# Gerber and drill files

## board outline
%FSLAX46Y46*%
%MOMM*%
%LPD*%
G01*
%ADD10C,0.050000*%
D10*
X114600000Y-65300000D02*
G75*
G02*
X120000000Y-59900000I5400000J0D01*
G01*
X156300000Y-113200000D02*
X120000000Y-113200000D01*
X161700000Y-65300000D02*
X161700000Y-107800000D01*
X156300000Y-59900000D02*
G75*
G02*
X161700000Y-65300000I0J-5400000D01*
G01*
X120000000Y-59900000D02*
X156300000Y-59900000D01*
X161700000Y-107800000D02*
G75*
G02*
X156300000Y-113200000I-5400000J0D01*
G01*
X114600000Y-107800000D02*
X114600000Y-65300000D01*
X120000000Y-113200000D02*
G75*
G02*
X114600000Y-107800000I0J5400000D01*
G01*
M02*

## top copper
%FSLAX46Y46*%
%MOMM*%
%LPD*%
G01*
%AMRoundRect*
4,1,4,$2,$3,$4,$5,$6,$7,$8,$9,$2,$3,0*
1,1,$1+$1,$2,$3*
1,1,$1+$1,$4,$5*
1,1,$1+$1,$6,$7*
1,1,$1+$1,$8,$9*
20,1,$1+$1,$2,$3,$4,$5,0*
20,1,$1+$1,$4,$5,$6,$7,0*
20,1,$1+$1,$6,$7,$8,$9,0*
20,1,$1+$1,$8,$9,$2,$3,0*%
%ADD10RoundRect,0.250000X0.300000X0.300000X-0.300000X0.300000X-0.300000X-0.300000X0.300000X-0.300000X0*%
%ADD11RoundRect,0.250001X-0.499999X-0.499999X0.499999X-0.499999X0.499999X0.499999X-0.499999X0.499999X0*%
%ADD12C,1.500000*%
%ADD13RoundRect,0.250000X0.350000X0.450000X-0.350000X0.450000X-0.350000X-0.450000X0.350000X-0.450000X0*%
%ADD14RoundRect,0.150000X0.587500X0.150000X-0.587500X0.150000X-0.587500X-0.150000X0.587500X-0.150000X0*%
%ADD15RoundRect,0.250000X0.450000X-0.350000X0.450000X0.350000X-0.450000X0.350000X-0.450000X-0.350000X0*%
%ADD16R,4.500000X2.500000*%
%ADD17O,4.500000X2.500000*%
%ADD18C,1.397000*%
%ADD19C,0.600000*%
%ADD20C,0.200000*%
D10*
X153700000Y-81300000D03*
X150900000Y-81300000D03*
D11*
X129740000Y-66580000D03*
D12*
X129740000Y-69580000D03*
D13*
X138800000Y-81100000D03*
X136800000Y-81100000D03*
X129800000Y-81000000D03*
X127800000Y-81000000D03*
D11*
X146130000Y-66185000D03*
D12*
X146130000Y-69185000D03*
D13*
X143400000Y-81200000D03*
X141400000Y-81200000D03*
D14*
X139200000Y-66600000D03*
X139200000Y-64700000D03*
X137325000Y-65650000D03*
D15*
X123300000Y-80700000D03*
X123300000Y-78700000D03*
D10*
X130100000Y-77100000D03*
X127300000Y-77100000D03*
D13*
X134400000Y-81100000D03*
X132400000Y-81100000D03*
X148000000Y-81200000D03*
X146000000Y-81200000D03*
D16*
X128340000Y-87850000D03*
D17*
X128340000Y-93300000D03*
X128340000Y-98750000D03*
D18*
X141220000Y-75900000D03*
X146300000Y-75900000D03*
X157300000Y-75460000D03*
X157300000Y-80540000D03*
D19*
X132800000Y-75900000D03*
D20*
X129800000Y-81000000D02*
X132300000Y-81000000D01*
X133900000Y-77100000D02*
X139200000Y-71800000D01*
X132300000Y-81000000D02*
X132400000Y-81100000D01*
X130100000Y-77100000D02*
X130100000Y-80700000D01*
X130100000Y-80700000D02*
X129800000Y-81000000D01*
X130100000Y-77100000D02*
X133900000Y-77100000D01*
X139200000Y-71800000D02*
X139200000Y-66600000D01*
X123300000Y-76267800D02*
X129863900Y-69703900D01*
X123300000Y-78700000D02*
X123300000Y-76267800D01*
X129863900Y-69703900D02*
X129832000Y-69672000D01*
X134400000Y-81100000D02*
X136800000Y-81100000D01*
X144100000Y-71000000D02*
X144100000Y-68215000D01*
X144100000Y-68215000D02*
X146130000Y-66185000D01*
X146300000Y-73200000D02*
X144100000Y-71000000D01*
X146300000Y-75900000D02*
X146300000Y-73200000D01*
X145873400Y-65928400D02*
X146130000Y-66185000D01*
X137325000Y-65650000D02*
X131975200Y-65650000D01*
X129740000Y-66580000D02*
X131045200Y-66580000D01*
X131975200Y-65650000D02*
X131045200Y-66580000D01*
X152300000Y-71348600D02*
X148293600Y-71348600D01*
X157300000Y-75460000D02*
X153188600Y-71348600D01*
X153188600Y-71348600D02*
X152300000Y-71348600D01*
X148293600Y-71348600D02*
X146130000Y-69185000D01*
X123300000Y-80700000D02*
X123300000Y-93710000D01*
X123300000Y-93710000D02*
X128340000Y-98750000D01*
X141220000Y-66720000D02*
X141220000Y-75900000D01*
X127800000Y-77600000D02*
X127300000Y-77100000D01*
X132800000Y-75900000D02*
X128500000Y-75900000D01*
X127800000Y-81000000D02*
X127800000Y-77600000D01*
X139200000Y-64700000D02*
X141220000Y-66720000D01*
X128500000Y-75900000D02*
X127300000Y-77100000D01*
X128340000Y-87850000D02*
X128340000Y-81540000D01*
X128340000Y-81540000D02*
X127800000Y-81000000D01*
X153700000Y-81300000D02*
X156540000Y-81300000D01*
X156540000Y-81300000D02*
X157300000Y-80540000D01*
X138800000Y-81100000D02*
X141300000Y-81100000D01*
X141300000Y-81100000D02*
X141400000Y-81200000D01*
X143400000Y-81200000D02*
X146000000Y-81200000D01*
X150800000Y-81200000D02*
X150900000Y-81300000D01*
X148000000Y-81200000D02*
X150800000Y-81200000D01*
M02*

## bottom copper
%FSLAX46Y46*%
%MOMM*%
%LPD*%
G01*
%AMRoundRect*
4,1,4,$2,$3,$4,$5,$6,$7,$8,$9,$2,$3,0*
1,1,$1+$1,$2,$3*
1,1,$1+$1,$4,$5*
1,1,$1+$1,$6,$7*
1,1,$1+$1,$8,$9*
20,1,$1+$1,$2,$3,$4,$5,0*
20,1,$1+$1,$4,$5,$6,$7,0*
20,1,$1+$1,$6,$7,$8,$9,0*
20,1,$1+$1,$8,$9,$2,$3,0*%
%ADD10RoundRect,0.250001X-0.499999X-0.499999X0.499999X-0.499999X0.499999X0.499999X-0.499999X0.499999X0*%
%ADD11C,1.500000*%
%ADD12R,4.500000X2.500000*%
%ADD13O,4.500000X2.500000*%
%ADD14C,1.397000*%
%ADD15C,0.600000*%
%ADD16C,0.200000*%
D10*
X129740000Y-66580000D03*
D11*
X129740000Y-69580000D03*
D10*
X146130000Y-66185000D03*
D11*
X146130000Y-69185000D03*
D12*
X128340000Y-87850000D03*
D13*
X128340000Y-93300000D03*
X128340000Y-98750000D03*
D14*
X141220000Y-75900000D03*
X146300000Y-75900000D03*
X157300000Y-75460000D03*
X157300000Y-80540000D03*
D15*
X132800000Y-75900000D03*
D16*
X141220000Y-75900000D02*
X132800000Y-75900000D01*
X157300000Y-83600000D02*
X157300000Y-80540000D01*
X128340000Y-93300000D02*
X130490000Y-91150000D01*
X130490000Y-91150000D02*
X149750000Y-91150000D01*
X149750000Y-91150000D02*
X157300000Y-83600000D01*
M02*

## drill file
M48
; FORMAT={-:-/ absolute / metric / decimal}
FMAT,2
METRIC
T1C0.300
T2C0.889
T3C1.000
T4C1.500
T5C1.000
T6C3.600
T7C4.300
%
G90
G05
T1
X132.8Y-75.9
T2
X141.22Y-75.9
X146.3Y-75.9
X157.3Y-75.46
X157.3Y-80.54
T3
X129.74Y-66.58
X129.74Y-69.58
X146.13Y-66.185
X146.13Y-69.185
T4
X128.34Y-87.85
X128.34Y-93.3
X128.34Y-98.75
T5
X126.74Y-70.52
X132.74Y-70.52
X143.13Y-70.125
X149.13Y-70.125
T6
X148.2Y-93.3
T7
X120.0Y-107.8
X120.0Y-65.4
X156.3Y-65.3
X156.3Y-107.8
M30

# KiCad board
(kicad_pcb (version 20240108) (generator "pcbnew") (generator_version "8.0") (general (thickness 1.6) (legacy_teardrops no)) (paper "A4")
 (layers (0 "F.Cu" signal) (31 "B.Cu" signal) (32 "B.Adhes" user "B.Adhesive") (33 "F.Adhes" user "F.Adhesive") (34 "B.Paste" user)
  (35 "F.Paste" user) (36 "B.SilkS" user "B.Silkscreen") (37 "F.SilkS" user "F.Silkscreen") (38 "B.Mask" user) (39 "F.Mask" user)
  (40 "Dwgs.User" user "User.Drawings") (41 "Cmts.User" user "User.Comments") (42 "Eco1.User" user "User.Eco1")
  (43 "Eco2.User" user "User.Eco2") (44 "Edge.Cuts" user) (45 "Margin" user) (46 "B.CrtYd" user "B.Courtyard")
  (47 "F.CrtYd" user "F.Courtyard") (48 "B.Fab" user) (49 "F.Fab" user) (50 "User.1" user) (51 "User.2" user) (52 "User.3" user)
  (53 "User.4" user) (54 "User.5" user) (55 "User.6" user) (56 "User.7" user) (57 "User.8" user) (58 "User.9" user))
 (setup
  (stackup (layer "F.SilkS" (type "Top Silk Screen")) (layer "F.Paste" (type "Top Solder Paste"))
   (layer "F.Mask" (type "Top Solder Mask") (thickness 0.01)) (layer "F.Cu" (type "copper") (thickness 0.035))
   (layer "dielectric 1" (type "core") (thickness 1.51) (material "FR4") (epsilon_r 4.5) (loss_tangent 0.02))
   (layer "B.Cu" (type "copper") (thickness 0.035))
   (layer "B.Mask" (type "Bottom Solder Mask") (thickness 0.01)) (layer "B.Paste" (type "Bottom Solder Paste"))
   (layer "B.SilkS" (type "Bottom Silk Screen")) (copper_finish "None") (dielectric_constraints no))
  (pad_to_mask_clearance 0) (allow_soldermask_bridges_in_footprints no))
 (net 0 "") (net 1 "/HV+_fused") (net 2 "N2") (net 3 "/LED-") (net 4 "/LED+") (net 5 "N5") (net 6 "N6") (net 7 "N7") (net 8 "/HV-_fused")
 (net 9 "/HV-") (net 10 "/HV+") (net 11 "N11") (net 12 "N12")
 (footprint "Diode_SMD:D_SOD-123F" (layer "F.Cu") (at 152.3 81.3 180)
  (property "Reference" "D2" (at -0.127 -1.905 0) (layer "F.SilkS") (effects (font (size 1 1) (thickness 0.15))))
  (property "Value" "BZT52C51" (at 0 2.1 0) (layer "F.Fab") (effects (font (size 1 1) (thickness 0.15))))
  (pad "1" smd roundrect (at -1.4 0 180) (size 1.1 1.1) (layers "F.Cu" "F.Paste" "F.Mask") (roundrect_rratio 0.2272727273)
   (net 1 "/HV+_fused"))
  (pad "2" smd roundrect (at 1.4 0 180) (size 1.1 1.1) (layers "F.Cu" "F.Paste" "F.Mask") (roundrect_rratio 0.2272727273) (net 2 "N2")))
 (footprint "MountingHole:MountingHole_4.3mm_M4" (layer "F.Cu") (at 119.999999 107.800001)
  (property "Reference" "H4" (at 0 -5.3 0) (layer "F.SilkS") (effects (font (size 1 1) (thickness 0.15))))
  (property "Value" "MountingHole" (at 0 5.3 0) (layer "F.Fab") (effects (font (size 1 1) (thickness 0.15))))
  (pad "" np_thru_hole circle (at 0 0) (size 4.3 4.3) (drill 4.3) (layers "*.Cu" "*.Mask")))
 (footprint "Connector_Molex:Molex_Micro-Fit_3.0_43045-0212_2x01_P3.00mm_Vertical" (layer "F.Cu") (at 129.74 66.58)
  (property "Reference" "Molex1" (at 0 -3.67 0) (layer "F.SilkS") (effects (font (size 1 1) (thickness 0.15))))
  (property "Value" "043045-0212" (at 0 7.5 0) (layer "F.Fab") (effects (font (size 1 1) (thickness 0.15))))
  (pad "" np_thru_hole circle (at -3 3.94) (size 1 1) (drill 1) (layers "*.Cu" "*.Mask"))
  (pad "" np_thru_hole circle (at 3 3.94) (size 1 1) (drill 1) (layers "*.Cu" "*.Mask"))
  (pad "1" thru_hole roundrect (at 0 0) (size 1.5 1.5) (drill 1) (layers "*.Cu" "*.Mask") (remove_unused_layers no)
   (roundrect_rratio 0.166667) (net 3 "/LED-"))
  (pad "2" thru_hole circle (at 0 3) (size 1.5 1.5) (drill 1) (layers "*.Cu" "*.Mask") (remove_unused_layers no) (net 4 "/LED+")))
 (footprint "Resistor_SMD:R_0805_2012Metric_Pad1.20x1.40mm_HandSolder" (layer "F.Cu") (at 137.8 81.1 180)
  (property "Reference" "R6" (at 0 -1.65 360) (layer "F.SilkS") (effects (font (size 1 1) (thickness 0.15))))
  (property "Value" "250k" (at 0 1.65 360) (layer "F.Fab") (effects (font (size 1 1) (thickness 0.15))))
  (pad "1" smd roundrect (at -1 0 180) (size 1.2 1.4) (layers "F.Cu" "F.Paste" "F.Mask") (roundrect_rratio 0.208333) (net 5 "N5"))
  (pad "2" smd roundrect (at 1 0 180) (size 1.2 1.4) (layers "F.Cu" "F.Paste" "F.Mask") (roundrect_rratio 0.208333) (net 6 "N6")))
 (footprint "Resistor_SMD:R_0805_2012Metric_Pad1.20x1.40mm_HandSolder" (layer "F.Cu") (at 128.8 81 180)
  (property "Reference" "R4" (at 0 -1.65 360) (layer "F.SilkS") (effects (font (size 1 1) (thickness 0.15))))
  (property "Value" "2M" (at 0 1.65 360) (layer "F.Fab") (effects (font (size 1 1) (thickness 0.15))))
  (pad "1" smd roundrect (at -1 0 180) (size 1.2 1.4) (layers "F.Cu" "F.Paste" "F.Mask") (roundrect_rratio 0.208333) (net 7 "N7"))
  (pad "2" smd roundrect (at 1 0 180) (size 1.2 1.4) (layers "F.Cu" "F.Paste" "F.Mask") (roundrect_rratio 0.208333) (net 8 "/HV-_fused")))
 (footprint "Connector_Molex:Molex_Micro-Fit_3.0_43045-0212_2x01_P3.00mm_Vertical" (layer "F.Cu") (at 146.13 66.185)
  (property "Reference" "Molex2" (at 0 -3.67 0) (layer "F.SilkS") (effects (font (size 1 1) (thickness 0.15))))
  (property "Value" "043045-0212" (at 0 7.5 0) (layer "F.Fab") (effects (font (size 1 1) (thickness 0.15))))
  (pad "" np_thru_hole circle (at -3 3.94) (size 1 1) (drill 1) (layers "*.Cu" "*.Mask"))
  (pad "" np_thru_hole circle (at 3 3.94) (size 1 1) (drill 1) (layers "*.Cu" "*.Mask"))
  (pad "1" thru_hole roundrect (at 0 0) (size 1.5 1.5) (drill 1) (layers "*.Cu" "*.Mask") (remove_unused_layers no)
   (roundrect_rratio 0.166667) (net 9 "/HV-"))
  (pad "2" thru_hole circle (at 0 3) (size 1.5 1.5) (drill 1) (layers "*.Cu" "*.Mask") (remove_unused_layers no) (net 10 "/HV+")))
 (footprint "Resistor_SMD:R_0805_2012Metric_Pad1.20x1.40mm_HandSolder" (layer "F.Cu") (at 142.4 81.2 180)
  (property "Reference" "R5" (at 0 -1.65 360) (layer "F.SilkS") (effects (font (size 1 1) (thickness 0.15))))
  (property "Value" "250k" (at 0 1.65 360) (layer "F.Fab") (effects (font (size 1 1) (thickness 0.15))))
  (pad "1" smd roundrect (at -1 0 180) (size 1.2 1.4) (layers "F.Cu" "F.Paste" "F.Mask") (roundrect_rratio 0.208333) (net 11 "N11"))
  (pad "2" smd roundrect (at 1 0 180) (size 1.2 1.4) (layers "F.Cu" "F.Paste" "F.Mask") (roundrect_rratio 0.208333) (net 5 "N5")))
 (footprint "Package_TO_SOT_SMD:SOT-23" (layer "F.Cu") (at 138.2625 65.65 180)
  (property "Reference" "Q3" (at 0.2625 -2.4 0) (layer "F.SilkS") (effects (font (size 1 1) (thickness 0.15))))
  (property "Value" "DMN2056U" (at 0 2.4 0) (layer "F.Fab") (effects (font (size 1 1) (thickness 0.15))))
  (pad "1" smd roundrect (at -0.9375 -0.95 180) (size 1.475 0.6) (layers "F.Cu" "F.Paste" "F.Mask") (roundrect_rratio 0.25) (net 7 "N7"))
  (pad "2" smd roundrect (at -0.9375 0.95 180) (size 1.475 0.6) (layers "F.Cu" "F.Paste" "F.Mask") (roundrect_rratio 0.25)
   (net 8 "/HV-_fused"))
  (pad "3" smd roundrect (at 0.9375 0 180) (size 1.475 0.6) (layers "F.Cu" "F.Paste" "F.Mask") (roundrect_rratio 0.25) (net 3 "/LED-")))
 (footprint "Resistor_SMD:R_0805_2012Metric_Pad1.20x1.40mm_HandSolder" (layer "F.Cu") (at 123.3 79.7 90)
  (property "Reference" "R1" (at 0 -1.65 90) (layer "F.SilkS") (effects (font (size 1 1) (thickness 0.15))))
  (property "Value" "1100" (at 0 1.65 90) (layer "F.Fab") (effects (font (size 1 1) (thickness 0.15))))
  (pad "1" smd roundrect (at -1 0 90) (size 1.2 1.4) (layers "F.Cu" "F.Paste" "F.Mask") (roundrect_rratio 0.208333) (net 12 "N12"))
  (pad "2" smd roundrect (at 1 0 90) (size 1.2 1.4) (layers "F.Cu" "F.Paste" "F.Mask") (roundrect_rratio 0.208333) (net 4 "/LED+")))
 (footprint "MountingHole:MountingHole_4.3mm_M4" (layer "F.Cu") (at 120 65.4)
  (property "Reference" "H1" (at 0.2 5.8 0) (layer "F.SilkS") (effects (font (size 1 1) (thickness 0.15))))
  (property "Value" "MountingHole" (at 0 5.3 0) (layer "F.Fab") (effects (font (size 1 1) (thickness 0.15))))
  (pad "" np_thru_hole circle (at 0 0) (size 4.3 4.3) (drill 4.3) (layers "*.Cu" "*.Mask")))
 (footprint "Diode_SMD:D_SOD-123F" (layer "F.Cu") (at 128.7 77.1 180)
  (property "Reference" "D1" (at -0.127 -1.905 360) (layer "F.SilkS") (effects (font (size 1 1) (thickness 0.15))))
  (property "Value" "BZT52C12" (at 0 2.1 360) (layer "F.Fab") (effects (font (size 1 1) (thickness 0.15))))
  (pad "1" smd roundrect (at -1.4 0 180) (size 1.1 1.1) (layers "F.Cu" "F.Paste" "F.Mask") (roundrect_rratio 0.2272727273) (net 7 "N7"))
  (pad "2" smd roundrect (at 1.4 0 180) (size 1.1 1.1) (layers "F.Cu" "F.Paste" "F.Mask") (roundrect_rratio 0.2272727273)
   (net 8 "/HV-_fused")))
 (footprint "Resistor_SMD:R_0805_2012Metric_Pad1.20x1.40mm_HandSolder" (layer "F.Cu") (at 133.4 81.1 180)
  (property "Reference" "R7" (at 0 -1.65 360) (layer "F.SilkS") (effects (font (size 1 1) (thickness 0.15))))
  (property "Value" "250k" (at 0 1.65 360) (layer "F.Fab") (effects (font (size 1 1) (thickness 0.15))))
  (pad "1" smd roundrect (at -1 0 180) (size 1.2 1.4) (layers "F.Cu" "F.Paste" "F.Mask") (roundrect_rratio 0.208333) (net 6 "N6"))
  (pad "2" smd roundrect (at 1 0 180) (size 1.2 1.4) (layers "F.Cu" "F.Paste" "F.Mask") (roundrect_rratio 0.208333) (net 7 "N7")))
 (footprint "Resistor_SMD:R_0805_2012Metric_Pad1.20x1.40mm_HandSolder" (layer "F.Cu") (at 147 81.2 180)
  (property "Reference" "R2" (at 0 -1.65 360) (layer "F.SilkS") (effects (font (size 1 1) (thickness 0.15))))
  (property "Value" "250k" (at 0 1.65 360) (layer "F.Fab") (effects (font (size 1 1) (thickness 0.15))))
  (pad "1" smd roundrect (at -1 0 180) (size 1.2 1.4) (layers "F.Cu" "F.Paste" "F.Mask") (roundrect_rratio 0.208333) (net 2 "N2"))
  (pad "2" smd roundrect (at 1 0 180) (size 1.2 1.4) (layers "F.Cu" "F.Paste" "F.Mask") (roundrect_rratio 0.208333) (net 11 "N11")))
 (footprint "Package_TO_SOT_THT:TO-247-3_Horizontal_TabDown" (layer "F.Cu") (at 128.34 87.85 -90)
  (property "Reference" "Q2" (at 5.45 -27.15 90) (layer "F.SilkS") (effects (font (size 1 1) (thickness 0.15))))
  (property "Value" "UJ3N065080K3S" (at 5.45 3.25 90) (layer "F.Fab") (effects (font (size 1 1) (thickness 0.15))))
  (pad "" np_thru_hole oval (at 5.45 -19.86 270) (size 3.6 3.6) (drill 3.6) (layers "*.Cu" "*.Mask"))
  (pad "1" thru_hole rect (at 0 0 270) (size 2.5 4.5) (drill 1.5) (layers "*.Cu" "*.Mask") (remove_unused_layers no) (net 8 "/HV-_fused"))
  (pad "2" thru_hole oval (at 5.45 0 270) (size 2.5 4.5) (drill 1.5) (layers "*.Cu" "*.Mask") (remove_unused_layers no) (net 1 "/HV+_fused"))
  (pad "3" thru_hole oval (at 10.9 0 270) (size 2.5 4.5) (drill 1.5) (layers "*.Cu" "*.Mask") (remove_unused_layers no) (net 12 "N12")))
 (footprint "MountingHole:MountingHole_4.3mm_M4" (layer "F.Cu") (at 156.300001 65.299999)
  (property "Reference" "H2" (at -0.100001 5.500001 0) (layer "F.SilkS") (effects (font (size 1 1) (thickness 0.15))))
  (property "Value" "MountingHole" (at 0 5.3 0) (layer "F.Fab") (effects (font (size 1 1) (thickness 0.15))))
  (pad "" np_thru_hole circle (at 0 0) (size 4.3 4.3) (drill 4.3) (layers "*.Cu" "*.Mask")))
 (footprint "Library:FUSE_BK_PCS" (layer "F.Cu") (at 143.76 75.9)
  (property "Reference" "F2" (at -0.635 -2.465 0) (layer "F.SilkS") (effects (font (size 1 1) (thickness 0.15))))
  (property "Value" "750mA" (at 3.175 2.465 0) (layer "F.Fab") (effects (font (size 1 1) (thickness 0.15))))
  (pad "1" thru_hole circle (at -2.54 0) (size 1.397 1.397) (drill 0.889) (layers "*.Cu" "*.Mask") (remove_unused_layers no)
   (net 8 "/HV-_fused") (solder_mask_margin 0.102))
  (pad "2" thru_hole circle (at 2.54 0) (size 1.397 1.397) (drill 0.889) (layers "*.Cu" "*.Mask") (remove_unused_layers no) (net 9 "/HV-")
   (solder_mask_margin 0.102)))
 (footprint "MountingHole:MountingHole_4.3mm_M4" (layer "F.Cu") (at 156.300001 107.800001)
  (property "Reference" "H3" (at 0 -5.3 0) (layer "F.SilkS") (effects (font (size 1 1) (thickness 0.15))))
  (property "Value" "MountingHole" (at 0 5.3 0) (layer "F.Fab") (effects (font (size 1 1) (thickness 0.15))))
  (pad "" np_thru_hole circle (at 0 0) (size 4.3 4.3) (drill 4.3) (layers "*.Cu" "*.Mask")))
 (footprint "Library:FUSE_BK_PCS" (layer "F.Cu") (at 157.3 78 -90)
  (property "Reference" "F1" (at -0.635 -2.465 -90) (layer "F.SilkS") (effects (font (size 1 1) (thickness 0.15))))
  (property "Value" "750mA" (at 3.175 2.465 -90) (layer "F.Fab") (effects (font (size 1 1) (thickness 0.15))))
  (pad "1" thru_hole circle (at -2.54 0 270) (size 1.397 1.397) (drill 0.889) (layers "*.Cu" "*.Mask") (remove_unused_layers no)
   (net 10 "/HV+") (solder_mask_margin 0.102))
  (pad "2" thru_hole circle (at 2.54 0 270) (size 1.397 1.397) (drill 0.889) (layers "*.Cu" "*.Mask") (remove_unused_layers no)
   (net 1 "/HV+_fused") (solder_mask_margin 0.102)))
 (gr_arc (start 114.6 65.3) (mid 116.181623 61.481623) (end 120 59.9) (stroke (width 0.05) (type default)) (layer "Edge.Cuts"))
 (gr_line (start 156.3 113.2) (end 120 113.2) (stroke (width 0.05) (type default)) (layer "Edge.Cuts"))
 (gr_line (start 161.7 65.3) (end 161.7 107.8) (stroke (width 0.05) (type default)) (layer "Edge.Cuts"))
 (gr_arc (start 156.3 59.9) (mid 160.118377 61.481623) (end 161.7 65.3) (stroke (width 0.05) (type default)) (layer "Edge.Cuts"))
 (gr_line (start 120 59.9) (end 156.3 59.9) (stroke (width 0.05) (type default)) (layer "Edge.Cuts"))
 (gr_arc (start 161.7 107.8) (mid 160.118377 111.618377) (end 156.3 113.2) (stroke (width 0.05) (type default)) (layer "Edge.Cuts"))
 (gr_line (start 114.6 107.8) (end 114.6 65.3) (stroke (width 0.05) (type default)) (layer "Edge.Cuts"))
 (gr_arc (start 120 113.2) (mid 116.181623 111.618377) (end 114.6 107.8) (stroke (width 0.05) (type default)) (layer "Edge.Cuts"))
 (segment (start 129.8 81) (end 132.3 81) (width 0.2) (layer "F.Cu") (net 7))
 (segment (start 133.9 77.1) (end 139.2 71.8) (width 0.2) (layer "F.Cu") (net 7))
 (segment (start 132.3 81) (end 132.4 81.1) (width 0.2) (layer "F.Cu") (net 7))
 (segment (start 130.1 77.1) (end 130.1 80.7) (width 0.2) (layer "F.Cu") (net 7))
 (segment (start 130.1 80.7) (end 129.8 81) (width 0.2) (layer "F.Cu") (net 7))
 (segment (start 130.1 77.1) (end 133.9 77.1) (width 0.2) (layer "F.Cu") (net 7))
 (segment (start 139.2 71.8) (end 139.2 66.6) (width 0.2) (layer "F.Cu") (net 7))
 (segment (start 123.3 76.2678) (end 129.8639 69.7039) (width 0.2) (layer "F.Cu") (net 4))
 (segment (start 123.3 78.7) (end 123.3 76.2678) (width 0.2) (layer "F.Cu") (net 4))
 (segment (start 129.8639 69.7039) (end 129.832 69.672) (width 0.2) (layer "F.Cu") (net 4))
 (segment (start 134.4 81.1) (end 136.8 81.1) (width 0.2) (layer "F.Cu") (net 6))
 (segment (start 144.1 71) (end 144.1 68.215) (width 0.2) (layer "F.Cu") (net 9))
 (segment (start 144.1 68.215) (end 146.13 66.185) (width 0.2) (layer "F.Cu") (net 9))
 (segment (start 146.3 73.2) (end 144.1 71) (width 0.2) (layer "F.Cu") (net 9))
 (segment (start 146.3 75.9) (end 146.3 73.2) (width 0.2) (layer "F.Cu") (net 9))
 (segment (start 145.8734 65.9284) (end 146.13 66.185) (width 0.2) (layer "F.Cu") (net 9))
 (segment (start 137.325 65.65) (end 131.9752 65.65) (width 0.2) (layer "F.Cu") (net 3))
 (segment (start 129.74 66.58) (end 131.0452 66.58) (width 0.2) (layer "F.Cu") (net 3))
 (segment (start 131.9752 65.65) (end 131.0452 66.58) (width 0.2) (layer "F.Cu") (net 3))
 (segment (start 152.3 71.3486) (end 148.2936 71.3486) (width 0.2) (layer "F.Cu") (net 10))
 (segment (start 157.3 75.46) (end 153.1886 71.3486) (width 0.2) (layer "F.Cu") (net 10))
 (segment (start 153.1886 71.3486) (end 152.3 71.3486) (width 0.2) (layer "F.Cu") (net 10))
 (segment (start 148.2936 71.3486) (end 146.13 69.185) (width 0.2) (layer "F.Cu") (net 10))
 (segment (start 123.3 80.7) (end 123.3 93.71) (width 0.2) (layer "F.Cu") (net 12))
 (segment (start 123.3 93.71) (end 128.34 98.75) (width 0.2) (layer "F.Cu") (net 12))
 (segment (start 141.22 66.72) (end 141.22 75.9) (width 0.2) (layer "F.Cu") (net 8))
 (segment (start 127.8 77.6) (end 127.3 77.1) (width 0.2) (layer "F.Cu") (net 8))
 (segment (start 132.8 75.9) (end 128.5 75.9) (width 0.2) (layer "F.Cu") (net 8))
 (segment (start 127.8 81) (end 127.8 77.6) (width 0.2) (layer "F.Cu") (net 8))
 (segment (start 139.2 64.7) (end 141.22 66.72) (width 0.2) (layer "F.Cu") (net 8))
 (segment (start 128.5 75.9) (end 127.3 77.1) (width 0.2) (layer "F.Cu") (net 8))
 (segment (start 128.34 87.85) (end 128.34 81.54) (width 0.2) (layer "F.Cu") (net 8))
 (segment (start 128.34 81.54) (end 127.8 81) (width 0.2) (layer "F.Cu") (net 8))
 (via (at 132.8 75.9) (size 0.6) (drill 0.3) (layers "F.Cu" "B.Cu") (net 8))
 (segment (start 141.22 75.9) (end 132.8 75.9) (width 0.2) (layer "B.Cu") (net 8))
 (segment (start 153.7 81.3) (end 156.54 81.3) (width 0.2) (layer "F.Cu") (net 1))
 (segment (start 156.54 81.3) (end 157.3 80.54) (width 0.2) (layer "F.Cu") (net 1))
 (segment (start 157.3 83.6) (end 157.3 80.54) (width 0.2) (layer "B.Cu") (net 1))
 (segment (start 128.34 93.3) (end 130.49 91.15) (width 0.2) (layer "B.Cu") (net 1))
 (segment (start 130.49 91.15) (end 149.75 91.15) (width 0.2) (layer "B.Cu") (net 1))
 (segment (start 149.75 91.15) (end 157.3 83.6) (width 0.2) (layer "B.Cu") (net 1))
 (segment (start 138.8 81.1) (end 141.3 81.1) (width 0.2) (layer "F.Cu") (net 5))
 (segment (start 141.3 81.1) (end 141.4 81.2) (width 0.2) (layer "F.Cu") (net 5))
 (segment (start 143.4 81.2) (end 146 81.2) (width 0.2) (layer "F.Cu") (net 11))
 (segment (start 150.8 81.2) (end 150.9 81.3) (width 0.2) (layer "F.Cu") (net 2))
 (segment (start 148 81.2) (end 150.8 81.2) (width 0.2) (layer "F.Cu") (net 2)))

